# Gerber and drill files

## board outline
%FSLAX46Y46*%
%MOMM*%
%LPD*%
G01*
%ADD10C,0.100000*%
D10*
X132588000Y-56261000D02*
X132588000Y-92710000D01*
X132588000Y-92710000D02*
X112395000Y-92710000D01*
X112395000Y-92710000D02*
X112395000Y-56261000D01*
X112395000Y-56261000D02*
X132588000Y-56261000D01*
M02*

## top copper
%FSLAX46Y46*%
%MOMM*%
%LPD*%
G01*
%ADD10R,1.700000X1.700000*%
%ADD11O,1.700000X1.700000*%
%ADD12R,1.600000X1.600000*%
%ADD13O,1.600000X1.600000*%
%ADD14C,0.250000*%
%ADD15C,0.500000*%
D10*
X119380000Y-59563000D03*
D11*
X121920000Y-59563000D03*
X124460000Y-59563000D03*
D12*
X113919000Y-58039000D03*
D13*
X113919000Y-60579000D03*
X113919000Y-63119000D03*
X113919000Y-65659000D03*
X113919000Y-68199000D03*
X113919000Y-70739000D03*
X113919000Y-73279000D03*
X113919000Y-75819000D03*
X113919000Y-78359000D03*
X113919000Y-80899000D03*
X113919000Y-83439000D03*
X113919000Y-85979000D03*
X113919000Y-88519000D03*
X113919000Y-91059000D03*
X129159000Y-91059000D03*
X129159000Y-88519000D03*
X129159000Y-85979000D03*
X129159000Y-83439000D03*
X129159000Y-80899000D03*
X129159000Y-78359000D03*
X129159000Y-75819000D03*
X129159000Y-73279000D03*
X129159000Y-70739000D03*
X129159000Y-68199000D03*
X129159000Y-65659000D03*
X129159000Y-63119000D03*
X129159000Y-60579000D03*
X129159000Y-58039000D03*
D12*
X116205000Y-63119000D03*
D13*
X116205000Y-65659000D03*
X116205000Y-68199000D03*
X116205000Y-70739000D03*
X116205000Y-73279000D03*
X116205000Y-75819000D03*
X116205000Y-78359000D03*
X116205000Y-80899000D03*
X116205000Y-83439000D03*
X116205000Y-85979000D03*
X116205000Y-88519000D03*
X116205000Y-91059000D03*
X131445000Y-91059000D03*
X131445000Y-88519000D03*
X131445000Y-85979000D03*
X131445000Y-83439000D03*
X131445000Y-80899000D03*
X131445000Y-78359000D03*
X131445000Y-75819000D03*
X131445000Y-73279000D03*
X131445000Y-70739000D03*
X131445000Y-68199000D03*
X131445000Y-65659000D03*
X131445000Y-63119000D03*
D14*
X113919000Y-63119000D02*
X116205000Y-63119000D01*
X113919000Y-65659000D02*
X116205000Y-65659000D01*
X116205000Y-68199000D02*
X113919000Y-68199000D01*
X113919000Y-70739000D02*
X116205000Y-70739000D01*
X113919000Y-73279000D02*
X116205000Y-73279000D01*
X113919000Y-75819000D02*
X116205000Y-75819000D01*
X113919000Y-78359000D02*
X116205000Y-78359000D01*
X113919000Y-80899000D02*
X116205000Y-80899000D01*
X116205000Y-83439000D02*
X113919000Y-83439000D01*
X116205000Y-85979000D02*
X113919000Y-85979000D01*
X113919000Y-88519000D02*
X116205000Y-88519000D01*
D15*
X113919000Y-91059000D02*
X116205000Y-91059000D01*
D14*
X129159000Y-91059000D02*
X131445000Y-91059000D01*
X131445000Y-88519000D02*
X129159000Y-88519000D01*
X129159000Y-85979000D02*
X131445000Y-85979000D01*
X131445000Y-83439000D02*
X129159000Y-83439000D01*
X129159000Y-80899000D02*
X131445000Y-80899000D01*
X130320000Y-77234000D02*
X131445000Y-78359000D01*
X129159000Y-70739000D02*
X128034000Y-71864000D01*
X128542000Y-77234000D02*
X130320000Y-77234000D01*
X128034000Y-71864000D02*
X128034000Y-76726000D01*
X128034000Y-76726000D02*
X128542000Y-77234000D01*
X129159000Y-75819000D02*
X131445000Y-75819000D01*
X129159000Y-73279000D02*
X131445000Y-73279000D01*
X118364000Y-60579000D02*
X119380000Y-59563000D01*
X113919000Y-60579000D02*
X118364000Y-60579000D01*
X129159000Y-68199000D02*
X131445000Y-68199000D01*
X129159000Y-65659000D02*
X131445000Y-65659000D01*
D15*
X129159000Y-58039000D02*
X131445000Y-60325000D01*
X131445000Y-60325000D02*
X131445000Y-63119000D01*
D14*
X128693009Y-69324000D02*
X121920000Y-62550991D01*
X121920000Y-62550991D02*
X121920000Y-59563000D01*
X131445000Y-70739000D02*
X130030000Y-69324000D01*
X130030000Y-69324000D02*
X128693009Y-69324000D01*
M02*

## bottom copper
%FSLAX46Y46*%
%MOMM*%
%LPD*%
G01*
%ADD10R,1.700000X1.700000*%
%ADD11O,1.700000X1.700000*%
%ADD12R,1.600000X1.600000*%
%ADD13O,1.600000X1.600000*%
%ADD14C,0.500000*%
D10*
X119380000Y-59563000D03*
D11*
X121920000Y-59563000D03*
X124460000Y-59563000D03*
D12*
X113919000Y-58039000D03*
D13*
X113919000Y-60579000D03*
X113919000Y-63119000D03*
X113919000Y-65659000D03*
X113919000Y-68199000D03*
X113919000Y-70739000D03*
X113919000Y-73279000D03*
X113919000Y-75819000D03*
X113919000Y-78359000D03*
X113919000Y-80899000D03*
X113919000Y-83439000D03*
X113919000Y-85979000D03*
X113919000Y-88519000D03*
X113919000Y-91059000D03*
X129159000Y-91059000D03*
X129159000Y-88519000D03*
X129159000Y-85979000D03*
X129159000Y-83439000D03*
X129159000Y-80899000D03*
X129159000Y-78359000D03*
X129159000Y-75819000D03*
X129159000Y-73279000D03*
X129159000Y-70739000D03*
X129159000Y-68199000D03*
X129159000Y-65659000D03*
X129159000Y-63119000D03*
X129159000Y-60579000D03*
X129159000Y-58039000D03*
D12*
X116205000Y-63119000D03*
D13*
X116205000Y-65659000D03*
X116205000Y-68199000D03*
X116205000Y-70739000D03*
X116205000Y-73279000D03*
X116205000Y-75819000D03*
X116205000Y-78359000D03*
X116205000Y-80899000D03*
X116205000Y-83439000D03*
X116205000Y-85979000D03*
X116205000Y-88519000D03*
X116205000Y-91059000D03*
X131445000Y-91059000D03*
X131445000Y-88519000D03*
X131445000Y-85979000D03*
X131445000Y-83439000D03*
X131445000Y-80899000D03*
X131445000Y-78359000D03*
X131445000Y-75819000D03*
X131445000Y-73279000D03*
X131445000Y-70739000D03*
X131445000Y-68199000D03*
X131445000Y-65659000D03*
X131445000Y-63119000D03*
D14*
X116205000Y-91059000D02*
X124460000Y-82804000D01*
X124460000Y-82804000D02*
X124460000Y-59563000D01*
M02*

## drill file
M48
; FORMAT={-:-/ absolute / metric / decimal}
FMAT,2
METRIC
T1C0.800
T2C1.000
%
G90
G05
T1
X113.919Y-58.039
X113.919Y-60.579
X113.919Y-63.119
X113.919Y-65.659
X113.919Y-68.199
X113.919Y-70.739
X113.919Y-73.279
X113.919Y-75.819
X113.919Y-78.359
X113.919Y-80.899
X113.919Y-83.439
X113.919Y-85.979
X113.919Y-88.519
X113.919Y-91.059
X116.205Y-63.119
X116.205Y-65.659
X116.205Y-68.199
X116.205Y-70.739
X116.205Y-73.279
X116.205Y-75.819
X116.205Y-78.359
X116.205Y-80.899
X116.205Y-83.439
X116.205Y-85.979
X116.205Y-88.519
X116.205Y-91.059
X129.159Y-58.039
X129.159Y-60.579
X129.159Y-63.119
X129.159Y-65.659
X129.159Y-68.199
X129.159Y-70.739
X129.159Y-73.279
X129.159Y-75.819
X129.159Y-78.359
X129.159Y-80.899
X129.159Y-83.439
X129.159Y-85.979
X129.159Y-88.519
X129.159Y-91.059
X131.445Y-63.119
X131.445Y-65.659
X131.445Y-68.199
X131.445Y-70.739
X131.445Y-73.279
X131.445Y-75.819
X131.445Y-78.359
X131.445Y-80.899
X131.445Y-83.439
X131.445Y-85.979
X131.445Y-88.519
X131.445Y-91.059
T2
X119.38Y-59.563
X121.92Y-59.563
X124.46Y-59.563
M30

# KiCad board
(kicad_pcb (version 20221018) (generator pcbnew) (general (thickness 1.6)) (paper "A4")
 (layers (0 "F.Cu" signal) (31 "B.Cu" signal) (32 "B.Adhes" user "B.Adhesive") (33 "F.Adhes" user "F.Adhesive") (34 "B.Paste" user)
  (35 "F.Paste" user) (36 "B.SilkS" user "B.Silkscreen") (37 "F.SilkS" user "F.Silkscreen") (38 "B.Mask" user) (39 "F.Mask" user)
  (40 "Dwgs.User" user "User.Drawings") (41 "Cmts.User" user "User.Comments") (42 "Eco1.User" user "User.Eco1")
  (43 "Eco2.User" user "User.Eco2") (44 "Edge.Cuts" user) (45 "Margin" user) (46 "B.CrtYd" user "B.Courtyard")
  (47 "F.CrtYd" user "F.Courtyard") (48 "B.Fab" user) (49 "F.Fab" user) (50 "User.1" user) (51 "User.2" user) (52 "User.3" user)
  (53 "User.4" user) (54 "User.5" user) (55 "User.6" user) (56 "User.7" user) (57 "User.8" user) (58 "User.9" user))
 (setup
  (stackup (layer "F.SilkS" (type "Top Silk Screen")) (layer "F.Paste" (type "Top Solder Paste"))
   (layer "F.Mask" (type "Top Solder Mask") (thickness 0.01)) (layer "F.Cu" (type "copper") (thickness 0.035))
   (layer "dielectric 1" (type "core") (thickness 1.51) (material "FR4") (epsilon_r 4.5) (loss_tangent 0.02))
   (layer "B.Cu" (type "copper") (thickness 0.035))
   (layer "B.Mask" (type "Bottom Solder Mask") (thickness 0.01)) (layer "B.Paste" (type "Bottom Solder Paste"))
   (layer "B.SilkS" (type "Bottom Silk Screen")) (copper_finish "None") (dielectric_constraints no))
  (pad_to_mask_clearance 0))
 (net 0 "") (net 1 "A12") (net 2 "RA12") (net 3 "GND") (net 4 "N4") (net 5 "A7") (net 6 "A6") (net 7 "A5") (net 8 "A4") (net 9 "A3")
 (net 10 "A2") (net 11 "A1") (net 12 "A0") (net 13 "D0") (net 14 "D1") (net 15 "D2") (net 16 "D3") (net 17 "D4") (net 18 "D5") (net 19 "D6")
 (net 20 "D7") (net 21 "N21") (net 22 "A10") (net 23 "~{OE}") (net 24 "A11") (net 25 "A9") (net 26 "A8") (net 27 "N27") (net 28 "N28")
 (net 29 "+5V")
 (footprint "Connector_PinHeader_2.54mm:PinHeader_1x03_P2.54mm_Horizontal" (layer "F.Cu") (at 119.38 59.563 90)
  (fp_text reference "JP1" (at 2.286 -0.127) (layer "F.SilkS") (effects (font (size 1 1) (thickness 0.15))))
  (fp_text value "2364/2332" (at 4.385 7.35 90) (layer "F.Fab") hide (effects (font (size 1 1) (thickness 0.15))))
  (pad "1" thru_hole rect (at 0 0 90) (size 1.7 1.7) (drill 1) (layers "*.Cu" "*.Mask") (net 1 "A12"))
  (pad "2" thru_hole oval (at 0 2.54 90) (size 1.7 1.7) (drill 1) (layers "*.Cu" "*.Mask") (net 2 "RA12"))
  (pad "3" thru_hole oval (at 0 5.08 90) (size 1.7 1.7) (drill 1) (layers "*.Cu" "*.Mask") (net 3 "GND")))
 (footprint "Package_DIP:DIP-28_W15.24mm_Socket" (layer "F.Cu") (at 113.919 58.039)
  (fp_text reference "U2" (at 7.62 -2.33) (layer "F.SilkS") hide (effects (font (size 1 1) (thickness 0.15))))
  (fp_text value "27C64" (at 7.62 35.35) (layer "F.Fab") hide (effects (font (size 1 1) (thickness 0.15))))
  (pad "1" thru_hole rect (at 0 0) (size 1.6 1.6) (drill 0.8) (layers "*.Cu" "*.Mask") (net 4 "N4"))
  (pad "2" thru_hole oval (at 0 2.54) (size 1.6 1.6) (drill 0.8) (layers "*.Cu" "*.Mask") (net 1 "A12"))
  (pad "3" thru_hole oval (at 0 5.08) (size 1.6 1.6) (drill 0.8) (layers "*.Cu" "*.Mask") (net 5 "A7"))
  (pad "4" thru_hole oval (at 0 7.62) (size 1.6 1.6) (drill 0.8) (layers "*.Cu" "*.Mask") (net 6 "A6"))
  (pad "5" thru_hole oval (at 0 10.16) (size 1.6 1.6) (drill 0.8) (layers "*.Cu" "*.Mask") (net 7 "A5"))
  (pad "6" thru_hole oval (at 0 12.7) (size 1.6 1.6) (drill 0.8) (layers "*.Cu" "*.Mask") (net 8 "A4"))
  (pad "7" thru_hole oval (at 0 15.24) (size 1.6 1.6) (drill 0.8) (layers "*.Cu" "*.Mask") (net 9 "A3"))
  (pad "8" thru_hole oval (at 0 17.78) (size 1.6 1.6) (drill 0.8) (layers "*.Cu" "*.Mask") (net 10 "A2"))
  (pad "9" thru_hole oval (at 0 20.32) (size 1.6 1.6) (drill 0.8) (layers "*.Cu" "*.Mask") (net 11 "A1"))
  (pad "10" thru_hole oval (at 0 22.86) (size 1.6 1.6) (drill 0.8) (layers "*.Cu" "*.Mask") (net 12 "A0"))
  (pad "11" thru_hole oval (at 0 25.4) (size 1.6 1.6) (drill 0.8) (layers "*.Cu" "*.Mask") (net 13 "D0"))
  (pad "12" thru_hole oval (at 0 27.94) (size 1.6 1.6) (drill 0.8) (layers "*.Cu" "*.Mask") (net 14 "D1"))
  (pad "13" thru_hole oval (at 0 30.48) (size 1.6 1.6) (drill 0.8) (layers "*.Cu" "*.Mask") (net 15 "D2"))
  (pad "14" thru_hole oval (at 0 33.02) (size 1.6 1.6) (drill 0.8) (layers "*.Cu" "*.Mask") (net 3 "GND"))
  (pad "15" thru_hole oval (at 15.24 33.02) (size 1.6 1.6) (drill 0.8) (layers "*.Cu" "*.Mask") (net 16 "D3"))
  (pad "16" thru_hole oval (at 15.24 30.48) (size 1.6 1.6) (drill 0.8) (layers "*.Cu" "*.Mask") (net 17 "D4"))
  (pad "17" thru_hole oval (at 15.24 27.94) (size 1.6 1.6) (drill 0.8) (layers "*.Cu" "*.Mask") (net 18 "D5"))
  (pad "18" thru_hole oval (at 15.24 25.4) (size 1.6 1.6) (drill 0.8) (layers "*.Cu" "*.Mask") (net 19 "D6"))
  (pad "19" thru_hole oval (at 15.24 22.86) (size 1.6 1.6) (drill 0.8) (layers "*.Cu" "*.Mask") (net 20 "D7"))
  (pad "20" thru_hole oval (at 15.24 20.32) (size 1.6 1.6) (drill 0.8) (layers "*.Cu" "*.Mask") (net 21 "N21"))
  (pad "21" thru_hole oval (at 15.24 17.78) (size 1.6 1.6) (drill 0.8) (layers "*.Cu" "*.Mask") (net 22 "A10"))
  (pad "22" thru_hole oval (at 15.24 15.24) (size 1.6 1.6) (drill 0.8) (layers "*.Cu" "*.Mask") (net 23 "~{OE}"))
  (pad "23" thru_hole oval (at 15.24 12.7) (size 1.6 1.6) (drill 0.8) (layers "*.Cu" "*.Mask") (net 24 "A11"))
  (pad "24" thru_hole oval (at 15.24 10.16) (size 1.6 1.6) (drill 0.8) (layers "*.Cu" "*.Mask") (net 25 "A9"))
  (pad "25" thru_hole oval (at 15.24 7.62) (size 1.6 1.6) (drill 0.8) (layers "*.Cu" "*.Mask") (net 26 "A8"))
  (pad "26" thru_hole oval (at 15.24 5.08) (size 1.6 1.6) (drill 0.8) (layers "*.Cu" "*.Mask") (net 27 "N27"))
  (pad "27" thru_hole oval (at 15.24 2.54) (size 1.6 1.6) (drill 0.8) (layers "*.Cu" "*.Mask") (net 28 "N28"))
  (pad "28" thru_hole oval (at 15.24 0) (size 1.6 1.6) (drill 0.8) (layers "*.Cu" "*.Mask") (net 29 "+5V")))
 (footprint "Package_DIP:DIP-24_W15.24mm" (layer "F.Cu") (at 116.205 63.119)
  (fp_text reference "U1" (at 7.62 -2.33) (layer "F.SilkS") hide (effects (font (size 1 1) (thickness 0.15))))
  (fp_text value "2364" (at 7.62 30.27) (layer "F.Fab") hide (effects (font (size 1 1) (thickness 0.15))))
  (pad "1" thru_hole rect (at 0 0) (size 1.6 1.6) (drill 0.8) (layers "*.Cu" "*.Mask") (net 5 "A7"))
  (pad "2" thru_hole oval (at 0 2.54) (size 1.6 1.6) (drill 0.8) (layers "*.Cu" "*.Mask") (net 6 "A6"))
  (pad "3" thru_hole oval (at 0 5.08) (size 1.6 1.6) (drill 0.8) (layers "*.Cu" "*.Mask") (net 7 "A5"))
  (pad "4" thru_hole oval (at 0 7.62) (size 1.6 1.6) (drill 0.8) (layers "*.Cu" "*.Mask") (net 8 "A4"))
  (pad "5" thru_hole oval (at 0 10.16) (size 1.6 1.6) (drill 0.8) (layers "*.Cu" "*.Mask") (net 9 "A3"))
  (pad "6" thru_hole oval (at 0 12.7) (size 1.6 1.6) (drill 0.8) (layers "*.Cu" "*.Mask") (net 10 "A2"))
  (pad "7" thru_hole oval (at 0 15.24) (size 1.6 1.6) (drill 0.8) (layers "*.Cu" "*.Mask") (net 11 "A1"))
  (pad "8" thru_hole oval (at 0 17.78) (size 1.6 1.6) (drill 0.8) (layers "*.Cu" "*.Mask") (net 12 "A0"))
  (pad "9" thru_hole oval (at 0 20.32) (size 1.6 1.6) (drill 0.8) (layers "*.Cu" "*.Mask") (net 13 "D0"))
  (pad "10" thru_hole oval (at 0 22.86) (size 1.6 1.6) (drill 0.8) (layers "*.Cu" "*.Mask") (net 14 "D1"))
  (pad "11" thru_hole oval (at 0 25.4) (size 1.6 1.6) (drill 0.8) (layers "*.Cu" "*.Mask") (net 15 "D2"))
  (pad "12" thru_hole oval (at 0 27.94) (size 1.6 1.6) (drill 0.8) (layers "*.Cu" "*.Mask") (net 3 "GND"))
  (pad "13" thru_hole oval (at 15.24 27.94) (size 1.6 1.6) (drill 0.8) (layers "*.Cu" "*.Mask") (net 16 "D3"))
  (pad "14" thru_hole oval (at 15.24 25.4) (size 1.6 1.6) (drill 0.8) (layers "*.Cu" "*.Mask") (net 17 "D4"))
  (pad "15" thru_hole oval (at 15.24 22.86) (size 1.6 1.6) (drill 0.8) (layers "*.Cu" "*.Mask") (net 18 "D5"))
  (pad "16" thru_hole oval (at 15.24 20.32) (size 1.6 1.6) (drill 0.8) (layers "*.Cu" "*.Mask") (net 19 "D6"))
  (pad "17" thru_hole oval (at 15.24 17.78) (size 1.6 1.6) (drill 0.8) (layers "*.Cu" "*.Mask") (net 20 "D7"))
  (pad "18" thru_hole oval (at 15.24 15.24) (size 1.6 1.6) (drill 0.8) (layers "*.Cu" "*.Mask") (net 24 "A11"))
  (pad "19" thru_hole oval (at 15.24 12.7) (size 1.6 1.6) (drill 0.8) (layers "*.Cu" "*.Mask") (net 22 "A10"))
  (pad "20" thru_hole oval (at 15.24 10.16) (size 1.6 1.6) (drill 0.8) (layers "*.Cu" "*.Mask") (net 23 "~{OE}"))
  (pad "21" thru_hole oval (at 15.24 7.62) (size 1.6 1.6) (drill 0.8) (layers "*.Cu" "*.Mask") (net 2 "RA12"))
  (pad "22" thru_hole oval (at 15.24 5.08) (size 1.6 1.6) (drill 0.8) (layers "*.Cu" "*.Mask") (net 25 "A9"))
  (pad "23" thru_hole oval (at 15.24 2.54) (size 1.6 1.6) (drill 0.8) (layers "*.Cu" "*.Mask") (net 26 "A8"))
  (pad "24" thru_hole oval (at 15.24 0) (size 1.6 1.6) (drill 0.8) (layers "*.Cu" "*.Mask") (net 29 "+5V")))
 (gr_line (start 132.588 56.261) (end 132.588 92.71) (stroke (width 0.1) (type default)) (layer "Edge.Cuts"))
 (gr_line (start 132.588 92.71) (end 112.395 92.71) (stroke (width 0.1) (type default)) (layer "Edge.Cuts"))
 (gr_line (start 112.395 92.71) (end 112.395 56.261) (stroke (width 0.1) (type default)) (layer "Edge.Cuts"))
 (gr_line (start 112.395 56.261) (end 132.588 56.261) (stroke (width 0.1) (type default)) (layer "Edge.Cuts"))
 (segment (start 113.919 63.119) (end 116.205 63.119) (width 0.25) (layer "F.Cu") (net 5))
 (segment (start 113.919 65.659) (end 116.205 65.659) (width 0.25) (layer "F.Cu") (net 6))
 (segment (start 116.205 68.199) (end 113.919 68.199) (width 0.25) (layer "F.Cu") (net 7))
 (segment (start 113.919 70.739) (end 116.205 70.739) (width 0.25) (layer "F.Cu") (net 8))
 (segment (start 113.919 73.279) (end 116.205 73.279) (width 0.25) (layer "F.Cu") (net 9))
 (segment (start 113.919 75.819) (end 116.205 75.819) (width 0.25) (layer "F.Cu") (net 10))
 (segment (start 113.919 78.359) (end 116.205 78.359) (width 0.25) (layer "F.Cu") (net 11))
 (segment (start 113.919 80.899) (end 116.205 80.899) (width 0.25) (layer "F.Cu") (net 12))
 (segment (start 116.205 83.439) (end 113.919 83.439) (width 0.25) (layer "F.Cu") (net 13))
 (segment (start 116.205 85.979) (end 113.919 85.979) (width 0.25) (layer "F.Cu") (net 14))
 (segment (start 113.919 88.519) (end 116.205 88.519) (width 0.25) (layer "F.Cu") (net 15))
 (segment (start 113.919 91.059) (end 116.205 91.059) (width 0.5) (layer "F.Cu") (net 3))
 (segment (start 116.205 91.059) (end 124.46 82.804) (width 0.5) (layer "B.Cu") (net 3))
 (segment (start 124.46 82.804) (end 124.46 59.563) (width 0.5) (layer "B.Cu") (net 3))
 (segment (start 129.159 91.059) (end 131.445 91.059) (width 0.25) (layer "F.Cu") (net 16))
 (segment (start 131.445 88.519) (end 129.159 88.519) (width 0.25) (layer "F.Cu") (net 17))
 (segment (start 129.159 85.979) (end 131.445 85.979) (width 0.25) (layer "F.Cu") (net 18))
 (segment (start 131.445 83.439) (end 129.159 83.439) (width 0.25) (layer "F.Cu") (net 19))
 (segment (start 129.159 80.899) (end 131.445 80.899) (width 0.25) (layer "F.Cu") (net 20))
 (segment (start 130.32 77.234) (end 131.445 78.359) (width 0.25) (layer "F.Cu") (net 24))
 (segment (start 129.159 70.739) (end 128.034 71.864) (width 0.25) (layer "F.Cu") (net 24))
 (segment (start 128.542 77.234) (end 130.32 77.234) (width 0.25) (layer "F.Cu") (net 24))
 (segment (start 128.034 71.864) (end 128.034 76.726) (width 0.25) (layer "F.Cu") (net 24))
 (segment (start 128.034 76.726) (end 128.542 77.234) (width 0.25) (layer "F.Cu") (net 24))
 (segment (start 129.159 75.819) (end 131.445 75.819) (width 0.25) (layer "F.Cu") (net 22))
 (segment (start 129.159 73.279) (end 131.445 73.279) (width 0.25) (layer "F.Cu") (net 23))
 (segment (start 118.364 60.579) (end 119.38 59.563) (width 0.25) (layer "F.Cu") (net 1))
 (segment (start 113.919 60.579) (end 118.364 60.579) (width 0.25) (layer "F.Cu") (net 1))
 (segment (start 129.159 68.199) (end 131.445 68.199) (width 0.25) (layer "F.Cu") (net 25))
 (segment (start 129.159 65.659) (end 131.445 65.659) (width 0.25) (layer "F.Cu") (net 26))
 (segment (start 129.159 58.039) (end 131.445 60.325) (width 0.5) (layer "F.Cu") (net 29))
 (segment (start 131.445 60.325) (end 131.445 63.119) (width 0.5) (layer "F.Cu") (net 29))
 (segment (start 128.693009 69.324) (end 121.92 62.550991) (width 0.25) (layer "F.Cu") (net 2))
 (segment (start 121.92 62.550991) (end 121.92 59.563) (width 0.25) (layer "F.Cu") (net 2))
 (segment (start 131.445 70.739) (end 130.03 69.324) (width 0.25) (layer "F.Cu") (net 2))
 (segment (start 130.03 69.324) (end 128.693009 69.324) (width 0.25) (layer "F.Cu") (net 2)))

